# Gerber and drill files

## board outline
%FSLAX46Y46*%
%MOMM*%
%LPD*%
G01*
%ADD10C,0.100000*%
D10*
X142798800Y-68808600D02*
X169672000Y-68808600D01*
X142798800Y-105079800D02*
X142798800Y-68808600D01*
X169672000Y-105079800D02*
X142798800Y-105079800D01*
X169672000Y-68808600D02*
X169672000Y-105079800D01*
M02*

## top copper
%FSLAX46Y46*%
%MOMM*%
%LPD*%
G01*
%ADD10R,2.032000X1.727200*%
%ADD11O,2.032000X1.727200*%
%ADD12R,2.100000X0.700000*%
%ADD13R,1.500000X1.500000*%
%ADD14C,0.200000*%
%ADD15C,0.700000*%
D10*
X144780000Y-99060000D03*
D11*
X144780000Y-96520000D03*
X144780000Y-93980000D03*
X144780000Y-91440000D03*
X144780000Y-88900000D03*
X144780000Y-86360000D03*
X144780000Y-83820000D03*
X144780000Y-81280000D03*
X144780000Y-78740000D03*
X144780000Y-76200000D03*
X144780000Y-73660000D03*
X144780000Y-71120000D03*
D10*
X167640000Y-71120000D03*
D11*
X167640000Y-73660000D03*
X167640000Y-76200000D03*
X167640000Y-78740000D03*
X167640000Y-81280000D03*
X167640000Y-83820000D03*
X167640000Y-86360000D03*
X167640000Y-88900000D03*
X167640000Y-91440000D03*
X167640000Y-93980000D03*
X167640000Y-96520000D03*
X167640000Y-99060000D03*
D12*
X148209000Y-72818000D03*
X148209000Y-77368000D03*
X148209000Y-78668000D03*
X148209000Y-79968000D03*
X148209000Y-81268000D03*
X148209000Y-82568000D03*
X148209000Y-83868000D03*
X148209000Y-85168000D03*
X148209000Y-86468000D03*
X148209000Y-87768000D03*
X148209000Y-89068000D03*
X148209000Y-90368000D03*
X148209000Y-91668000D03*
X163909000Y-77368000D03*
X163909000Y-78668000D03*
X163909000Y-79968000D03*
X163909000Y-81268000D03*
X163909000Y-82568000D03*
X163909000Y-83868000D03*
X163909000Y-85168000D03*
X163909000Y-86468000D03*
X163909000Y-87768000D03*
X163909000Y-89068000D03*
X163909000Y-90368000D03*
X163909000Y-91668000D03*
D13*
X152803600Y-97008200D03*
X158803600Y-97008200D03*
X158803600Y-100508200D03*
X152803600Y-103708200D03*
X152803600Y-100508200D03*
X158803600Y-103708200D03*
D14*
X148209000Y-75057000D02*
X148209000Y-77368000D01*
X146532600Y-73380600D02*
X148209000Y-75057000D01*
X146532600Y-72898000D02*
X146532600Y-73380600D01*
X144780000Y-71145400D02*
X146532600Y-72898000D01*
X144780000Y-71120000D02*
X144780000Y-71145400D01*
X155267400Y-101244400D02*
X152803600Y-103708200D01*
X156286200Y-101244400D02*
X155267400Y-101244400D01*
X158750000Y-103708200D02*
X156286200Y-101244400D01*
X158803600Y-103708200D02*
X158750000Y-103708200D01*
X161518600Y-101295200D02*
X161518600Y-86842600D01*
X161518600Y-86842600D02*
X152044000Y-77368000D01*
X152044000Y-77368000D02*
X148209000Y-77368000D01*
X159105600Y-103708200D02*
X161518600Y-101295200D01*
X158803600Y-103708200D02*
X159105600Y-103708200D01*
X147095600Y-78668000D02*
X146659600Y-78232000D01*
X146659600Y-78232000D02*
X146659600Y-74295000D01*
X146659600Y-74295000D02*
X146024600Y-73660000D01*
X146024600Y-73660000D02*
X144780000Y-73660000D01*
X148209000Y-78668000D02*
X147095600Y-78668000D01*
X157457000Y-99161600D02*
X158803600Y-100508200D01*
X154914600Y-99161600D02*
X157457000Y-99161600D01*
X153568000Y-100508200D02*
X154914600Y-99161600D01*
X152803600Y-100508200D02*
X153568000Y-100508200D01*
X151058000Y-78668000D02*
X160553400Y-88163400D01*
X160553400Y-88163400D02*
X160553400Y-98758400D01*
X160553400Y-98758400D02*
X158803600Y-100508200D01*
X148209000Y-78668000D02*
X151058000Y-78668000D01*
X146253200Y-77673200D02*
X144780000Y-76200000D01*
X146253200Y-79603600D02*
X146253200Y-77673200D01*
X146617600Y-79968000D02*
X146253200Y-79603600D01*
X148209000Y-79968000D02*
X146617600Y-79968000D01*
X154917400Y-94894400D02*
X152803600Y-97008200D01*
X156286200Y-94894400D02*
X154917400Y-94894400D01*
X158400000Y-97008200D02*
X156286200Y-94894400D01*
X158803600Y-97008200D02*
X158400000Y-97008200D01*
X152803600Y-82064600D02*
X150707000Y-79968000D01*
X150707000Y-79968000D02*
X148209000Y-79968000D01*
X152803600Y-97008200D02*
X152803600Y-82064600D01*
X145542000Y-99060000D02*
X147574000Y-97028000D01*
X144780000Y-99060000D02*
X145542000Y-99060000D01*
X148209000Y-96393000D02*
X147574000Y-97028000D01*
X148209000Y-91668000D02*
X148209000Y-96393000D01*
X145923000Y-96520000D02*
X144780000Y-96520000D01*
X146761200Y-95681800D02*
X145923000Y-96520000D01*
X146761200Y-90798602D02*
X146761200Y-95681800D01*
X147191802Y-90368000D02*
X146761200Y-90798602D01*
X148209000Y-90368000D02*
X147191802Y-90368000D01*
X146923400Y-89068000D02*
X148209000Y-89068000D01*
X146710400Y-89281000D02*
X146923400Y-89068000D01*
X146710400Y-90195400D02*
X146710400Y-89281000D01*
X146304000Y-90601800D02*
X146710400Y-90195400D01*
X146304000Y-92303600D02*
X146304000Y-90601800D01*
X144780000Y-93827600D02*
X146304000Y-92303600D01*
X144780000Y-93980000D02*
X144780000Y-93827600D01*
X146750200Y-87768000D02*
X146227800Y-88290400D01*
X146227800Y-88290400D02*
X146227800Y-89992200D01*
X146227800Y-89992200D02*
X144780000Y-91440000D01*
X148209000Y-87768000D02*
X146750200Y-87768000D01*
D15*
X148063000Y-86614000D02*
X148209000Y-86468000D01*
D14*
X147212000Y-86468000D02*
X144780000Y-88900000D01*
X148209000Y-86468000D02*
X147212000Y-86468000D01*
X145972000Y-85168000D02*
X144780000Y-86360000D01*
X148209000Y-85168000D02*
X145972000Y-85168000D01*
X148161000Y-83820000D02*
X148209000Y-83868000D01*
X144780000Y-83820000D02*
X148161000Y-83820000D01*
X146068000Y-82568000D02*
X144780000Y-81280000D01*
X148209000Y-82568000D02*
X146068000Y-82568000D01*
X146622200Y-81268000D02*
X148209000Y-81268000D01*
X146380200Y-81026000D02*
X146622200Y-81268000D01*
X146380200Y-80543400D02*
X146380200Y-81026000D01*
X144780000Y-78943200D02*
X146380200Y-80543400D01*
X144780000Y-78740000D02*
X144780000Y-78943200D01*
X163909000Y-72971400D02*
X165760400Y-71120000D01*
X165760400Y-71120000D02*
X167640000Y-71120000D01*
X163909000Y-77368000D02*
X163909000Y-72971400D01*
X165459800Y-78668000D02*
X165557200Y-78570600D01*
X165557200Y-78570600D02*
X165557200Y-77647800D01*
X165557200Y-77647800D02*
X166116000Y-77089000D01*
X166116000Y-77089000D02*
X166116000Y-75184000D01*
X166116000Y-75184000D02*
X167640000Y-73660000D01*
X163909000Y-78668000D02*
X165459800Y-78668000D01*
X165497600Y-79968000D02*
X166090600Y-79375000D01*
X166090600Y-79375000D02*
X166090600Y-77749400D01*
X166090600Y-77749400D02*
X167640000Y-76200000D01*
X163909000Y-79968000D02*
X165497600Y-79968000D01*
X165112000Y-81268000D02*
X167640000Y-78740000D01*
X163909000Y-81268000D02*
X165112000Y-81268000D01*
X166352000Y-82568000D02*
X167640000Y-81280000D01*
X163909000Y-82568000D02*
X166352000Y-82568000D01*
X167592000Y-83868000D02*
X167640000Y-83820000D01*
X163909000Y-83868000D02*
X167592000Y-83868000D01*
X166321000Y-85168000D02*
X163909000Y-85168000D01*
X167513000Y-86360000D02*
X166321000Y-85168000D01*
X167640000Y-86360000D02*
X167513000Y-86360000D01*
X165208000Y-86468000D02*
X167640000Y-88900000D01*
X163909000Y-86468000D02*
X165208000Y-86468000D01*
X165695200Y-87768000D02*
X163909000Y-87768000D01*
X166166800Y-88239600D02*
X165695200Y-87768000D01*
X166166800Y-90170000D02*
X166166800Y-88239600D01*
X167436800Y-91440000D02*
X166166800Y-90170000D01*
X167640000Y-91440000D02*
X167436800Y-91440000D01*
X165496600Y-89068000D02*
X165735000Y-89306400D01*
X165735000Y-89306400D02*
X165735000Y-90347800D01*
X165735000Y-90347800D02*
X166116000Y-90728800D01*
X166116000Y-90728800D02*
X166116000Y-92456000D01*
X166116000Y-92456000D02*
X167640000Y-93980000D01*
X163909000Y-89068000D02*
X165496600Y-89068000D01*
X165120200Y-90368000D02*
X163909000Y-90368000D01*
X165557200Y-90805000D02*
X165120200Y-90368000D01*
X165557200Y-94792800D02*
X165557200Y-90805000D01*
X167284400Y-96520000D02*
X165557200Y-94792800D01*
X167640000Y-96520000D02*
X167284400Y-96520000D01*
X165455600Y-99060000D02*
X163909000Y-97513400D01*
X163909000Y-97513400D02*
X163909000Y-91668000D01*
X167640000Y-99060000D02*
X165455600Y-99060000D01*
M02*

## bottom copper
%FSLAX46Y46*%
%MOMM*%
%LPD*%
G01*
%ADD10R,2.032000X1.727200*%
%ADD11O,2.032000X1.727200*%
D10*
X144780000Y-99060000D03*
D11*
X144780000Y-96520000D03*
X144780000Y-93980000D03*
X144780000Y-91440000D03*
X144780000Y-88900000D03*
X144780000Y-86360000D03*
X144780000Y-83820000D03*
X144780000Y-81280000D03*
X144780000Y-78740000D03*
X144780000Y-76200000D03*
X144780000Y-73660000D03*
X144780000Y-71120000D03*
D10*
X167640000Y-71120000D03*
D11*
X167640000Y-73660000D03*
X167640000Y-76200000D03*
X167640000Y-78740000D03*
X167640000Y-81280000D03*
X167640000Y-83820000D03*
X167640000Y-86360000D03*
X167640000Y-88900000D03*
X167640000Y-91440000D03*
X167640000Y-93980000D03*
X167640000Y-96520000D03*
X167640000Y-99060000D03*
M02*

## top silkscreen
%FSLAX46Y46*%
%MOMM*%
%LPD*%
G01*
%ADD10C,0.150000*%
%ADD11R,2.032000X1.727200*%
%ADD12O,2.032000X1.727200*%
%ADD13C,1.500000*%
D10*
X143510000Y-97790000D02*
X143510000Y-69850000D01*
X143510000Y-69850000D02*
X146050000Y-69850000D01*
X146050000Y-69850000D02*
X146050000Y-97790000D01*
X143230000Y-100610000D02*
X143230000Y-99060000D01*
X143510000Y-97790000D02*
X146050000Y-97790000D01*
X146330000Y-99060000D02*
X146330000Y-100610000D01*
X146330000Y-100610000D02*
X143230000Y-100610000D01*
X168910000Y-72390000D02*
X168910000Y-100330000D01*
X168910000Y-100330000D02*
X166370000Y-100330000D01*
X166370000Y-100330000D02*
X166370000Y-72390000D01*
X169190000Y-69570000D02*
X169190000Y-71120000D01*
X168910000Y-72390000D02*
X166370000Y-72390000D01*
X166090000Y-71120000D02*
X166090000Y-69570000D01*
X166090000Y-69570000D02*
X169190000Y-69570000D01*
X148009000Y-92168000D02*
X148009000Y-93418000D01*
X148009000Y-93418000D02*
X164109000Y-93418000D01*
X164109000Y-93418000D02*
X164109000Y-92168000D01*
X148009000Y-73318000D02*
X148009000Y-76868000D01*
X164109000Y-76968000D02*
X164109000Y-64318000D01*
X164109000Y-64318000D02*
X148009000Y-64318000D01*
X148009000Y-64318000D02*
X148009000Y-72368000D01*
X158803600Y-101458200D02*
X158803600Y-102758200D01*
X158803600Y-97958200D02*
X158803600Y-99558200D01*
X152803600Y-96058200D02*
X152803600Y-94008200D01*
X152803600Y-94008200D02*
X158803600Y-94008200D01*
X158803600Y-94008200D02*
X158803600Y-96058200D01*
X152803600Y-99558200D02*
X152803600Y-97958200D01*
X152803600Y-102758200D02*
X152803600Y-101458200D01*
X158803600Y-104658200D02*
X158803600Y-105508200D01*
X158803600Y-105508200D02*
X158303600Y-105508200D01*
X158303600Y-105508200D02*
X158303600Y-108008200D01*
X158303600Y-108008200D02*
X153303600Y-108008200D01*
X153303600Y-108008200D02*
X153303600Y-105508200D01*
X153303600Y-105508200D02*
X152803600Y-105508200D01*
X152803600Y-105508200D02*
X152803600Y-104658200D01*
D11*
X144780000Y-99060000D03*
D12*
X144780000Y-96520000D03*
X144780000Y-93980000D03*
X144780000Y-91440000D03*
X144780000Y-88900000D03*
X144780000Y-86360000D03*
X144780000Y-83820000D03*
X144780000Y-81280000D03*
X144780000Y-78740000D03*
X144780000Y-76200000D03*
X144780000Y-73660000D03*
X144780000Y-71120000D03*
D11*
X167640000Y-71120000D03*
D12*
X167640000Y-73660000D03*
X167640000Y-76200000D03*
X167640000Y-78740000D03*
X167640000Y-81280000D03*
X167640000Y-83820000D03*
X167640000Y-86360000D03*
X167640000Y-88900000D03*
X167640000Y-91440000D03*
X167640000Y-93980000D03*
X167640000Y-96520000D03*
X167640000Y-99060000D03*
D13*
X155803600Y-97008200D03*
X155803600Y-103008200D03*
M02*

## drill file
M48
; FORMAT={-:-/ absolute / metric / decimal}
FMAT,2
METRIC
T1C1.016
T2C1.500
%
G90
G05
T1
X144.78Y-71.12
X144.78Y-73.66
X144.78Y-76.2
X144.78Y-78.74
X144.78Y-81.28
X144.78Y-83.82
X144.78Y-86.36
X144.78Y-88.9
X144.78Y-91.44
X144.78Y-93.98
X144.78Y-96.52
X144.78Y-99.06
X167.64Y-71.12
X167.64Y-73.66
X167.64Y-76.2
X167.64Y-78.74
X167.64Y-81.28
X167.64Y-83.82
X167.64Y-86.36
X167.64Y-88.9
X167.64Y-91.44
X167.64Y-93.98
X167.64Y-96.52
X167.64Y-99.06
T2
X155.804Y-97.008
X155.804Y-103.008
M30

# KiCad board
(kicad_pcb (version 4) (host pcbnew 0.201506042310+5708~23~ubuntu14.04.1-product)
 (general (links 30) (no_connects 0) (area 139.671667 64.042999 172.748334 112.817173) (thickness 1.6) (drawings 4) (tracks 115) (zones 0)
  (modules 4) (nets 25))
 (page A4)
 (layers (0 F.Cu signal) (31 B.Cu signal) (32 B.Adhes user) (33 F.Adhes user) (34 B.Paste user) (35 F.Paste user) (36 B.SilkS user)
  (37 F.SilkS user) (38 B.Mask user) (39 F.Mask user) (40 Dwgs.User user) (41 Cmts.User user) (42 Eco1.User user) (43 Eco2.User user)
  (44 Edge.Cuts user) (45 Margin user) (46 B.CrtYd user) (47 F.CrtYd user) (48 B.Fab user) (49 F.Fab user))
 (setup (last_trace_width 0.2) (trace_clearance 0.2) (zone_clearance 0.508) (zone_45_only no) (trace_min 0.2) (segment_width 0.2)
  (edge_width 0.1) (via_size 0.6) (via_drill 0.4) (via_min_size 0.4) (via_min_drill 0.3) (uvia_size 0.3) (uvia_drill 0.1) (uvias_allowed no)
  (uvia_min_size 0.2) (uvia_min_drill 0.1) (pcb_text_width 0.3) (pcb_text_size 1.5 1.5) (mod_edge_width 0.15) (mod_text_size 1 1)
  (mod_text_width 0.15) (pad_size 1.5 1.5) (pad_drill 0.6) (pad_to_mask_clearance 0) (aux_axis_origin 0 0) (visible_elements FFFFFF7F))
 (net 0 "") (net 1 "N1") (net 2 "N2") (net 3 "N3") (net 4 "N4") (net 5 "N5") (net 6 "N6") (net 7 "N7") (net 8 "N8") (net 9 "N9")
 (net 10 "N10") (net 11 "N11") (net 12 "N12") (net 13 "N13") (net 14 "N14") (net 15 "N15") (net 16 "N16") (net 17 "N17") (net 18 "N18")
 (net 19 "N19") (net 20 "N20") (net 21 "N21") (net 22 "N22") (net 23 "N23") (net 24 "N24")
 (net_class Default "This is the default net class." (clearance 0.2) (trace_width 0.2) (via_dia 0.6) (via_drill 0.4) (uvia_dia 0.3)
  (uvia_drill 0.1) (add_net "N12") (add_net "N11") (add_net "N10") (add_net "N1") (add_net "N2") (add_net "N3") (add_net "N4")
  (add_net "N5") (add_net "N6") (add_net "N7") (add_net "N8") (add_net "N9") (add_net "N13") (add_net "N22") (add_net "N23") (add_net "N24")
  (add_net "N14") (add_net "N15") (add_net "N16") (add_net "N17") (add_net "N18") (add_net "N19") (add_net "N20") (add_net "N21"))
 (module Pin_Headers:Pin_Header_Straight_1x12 (layer F.Cu) (at 144.78 99.06 180)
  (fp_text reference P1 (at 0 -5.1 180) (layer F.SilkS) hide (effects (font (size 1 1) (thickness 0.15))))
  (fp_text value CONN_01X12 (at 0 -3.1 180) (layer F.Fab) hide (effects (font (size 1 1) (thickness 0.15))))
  (fp_line (start 1.27 1.27) (end 1.27 29.21) (layer F.SilkS) (width 0.15))
  (fp_line (start 1.27 29.21) (end -1.27 29.21) (layer F.SilkS) (width 0.15))
  (fp_line (start -1.27 29.21) (end -1.27 1.27) (layer F.SilkS) (width 0.15))
  (fp_line (start 1.55 -1.55) (end 1.55 0) (layer F.SilkS) (width 0.15))
  (fp_line (start 1.27 1.27) (end -1.27 1.27) (layer F.SilkS) (width 0.15))
  (fp_line (start -1.55 0) (end -1.55 -1.55) (layer F.SilkS) (width 0.15))
  (fp_line (start -1.55 -1.55) (end 1.55 -1.55) (layer F.SilkS) (width 0.15))
  (pad 1 thru_hole rect (at 0 0 180) (size 2.032 1.7272) (drill 1.016) (layers *.Cu *.Mask F.SilkS) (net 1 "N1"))
  (pad 2 thru_hole oval (at 0 2.54 180) (size 2.032 1.7272) (drill 1.016) (layers *.Cu *.Mask F.SilkS) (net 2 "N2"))
  (pad 3 thru_hole oval (at 0 5.08 180) (size 2.032 1.7272) (drill 1.016) (layers *.Cu *.Mask F.SilkS) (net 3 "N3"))
  (pad 4 thru_hole oval (at 0 7.62 180) (size 2.032 1.7272) (drill 1.016) (layers *.Cu *.Mask F.SilkS) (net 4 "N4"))
  (pad 5 thru_hole oval (at 0 10.16 180) (size 2.032 1.7272) (drill 1.016) (layers *.Cu *.Mask F.SilkS) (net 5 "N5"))
  (pad 6 thru_hole oval (at 0 12.7 180) (size 2.032 1.7272) (drill 1.016) (layers *.Cu *.Mask F.SilkS) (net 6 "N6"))
  (pad 7 thru_hole oval (at 0 15.24 180) (size 2.032 1.7272) (drill 1.016) (layers *.Cu *.Mask F.SilkS) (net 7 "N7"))
  (pad 8 thru_hole oval (at 0 17.78 180) (size 2.032 1.7272) (drill 1.016) (layers *.Cu *.Mask F.SilkS) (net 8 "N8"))
  (pad 9 thru_hole oval (at 0 20.32 180) (size 2.032 1.7272) (drill 1.016) (layers *.Cu *.Mask F.SilkS) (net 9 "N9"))
  (pad 10 thru_hole oval (at 0 22.86 180) (size 2.032 1.7272) (drill 1.016) (layers *.Cu *.Mask F.SilkS) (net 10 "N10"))
  (pad 11 thru_hole oval (at 0 25.4 180) (size 2.032 1.7272) (drill 1.016) (layers *.Cu *.Mask F.SilkS) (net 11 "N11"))
  (pad 12 thru_hole oval (at 0 27.94 180) (size 2.032 1.7272) (drill 1.016) (layers *.Cu *.Mask F.SilkS) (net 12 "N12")))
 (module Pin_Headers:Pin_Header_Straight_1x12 (layer F.Cu) (at 167.64 71.12)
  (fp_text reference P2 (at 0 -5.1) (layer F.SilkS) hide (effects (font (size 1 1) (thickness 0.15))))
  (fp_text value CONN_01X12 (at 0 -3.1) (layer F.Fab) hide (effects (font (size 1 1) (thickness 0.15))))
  (fp_line (start 1.27 1.27) (end 1.27 29.21) (layer F.SilkS) (width 0.15))
  (fp_line (start 1.27 29.21) (end -1.27 29.21) (layer F.SilkS) (width 0.15))
  (fp_line (start -1.27 29.21) (end -1.27 1.27) (layer F.SilkS) (width 0.15))
  (fp_line (start 1.55 -1.55) (end 1.55 0) (layer F.SilkS) (width 0.15))
  (fp_line (start 1.27 1.27) (end -1.27 1.27) (layer F.SilkS) (width 0.15))
  (fp_line (start -1.55 0) (end -1.55 -1.55) (layer F.SilkS) (width 0.15))
  (fp_line (start -1.55 -1.55) (end 1.55 -1.55) (layer F.SilkS) (width 0.15))
  (pad 1 thru_hole rect (at 0 0) (size 2.032 1.7272) (drill 1.016) (layers *.Cu *.Mask F.SilkS) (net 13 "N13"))
  (pad 2 thru_hole oval (at 0 2.54) (size 2.032 1.7272) (drill 1.016) (layers *.Cu *.Mask F.SilkS) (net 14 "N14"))
  (pad 3 thru_hole oval (at 0 5.08) (size 2.032 1.7272) (drill 1.016) (layers *.Cu *.Mask F.SilkS) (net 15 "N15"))
  (pad 4 thru_hole oval (at 0 7.62) (size 2.032 1.7272) (drill 1.016) (layers *.Cu *.Mask F.SilkS) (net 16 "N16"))
  (pad 5 thru_hole oval (at 0 10.16) (size 2.032 1.7272) (drill 1.016) (layers *.Cu *.Mask F.SilkS) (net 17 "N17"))
  (pad 6 thru_hole oval (at 0 12.7) (size 2.032 1.7272) (drill 1.016) (layers *.Cu *.Mask F.SilkS) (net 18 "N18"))
  (pad 7 thru_hole oval (at 0 15.24) (size 2.032 1.7272) (drill 1.016) (layers *.Cu *.Mask F.SilkS) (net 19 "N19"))
  (pad 8 thru_hole oval (at 0 17.78) (size 2.032 1.7272) (drill 1.016) (layers *.Cu *.Mask F.SilkS) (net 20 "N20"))
  (pad 9 thru_hole oval (at 0 20.32) (size 2.032 1.7272) (drill 1.016) (layers *.Cu *.Mask F.SilkS) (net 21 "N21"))
  (pad 10 thru_hole oval (at 0 22.86) (size 2.032 1.7272) (drill 1.016) (layers *.Cu *.Mask F.SilkS) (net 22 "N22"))
  (pad 11 thru_hole oval (at 0 25.4) (size 2.032 1.7272) (drill 1.016) (layers *.Cu *.Mask F.SilkS) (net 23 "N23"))
  (pad 12 thru_hole oval (at 0 27.94) (size 2.032 1.7272) (drill 1.016) (layers *.Cu *.Mask F.SilkS) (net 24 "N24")))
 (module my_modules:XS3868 (layer F.Cu) (at 148.209 93.218)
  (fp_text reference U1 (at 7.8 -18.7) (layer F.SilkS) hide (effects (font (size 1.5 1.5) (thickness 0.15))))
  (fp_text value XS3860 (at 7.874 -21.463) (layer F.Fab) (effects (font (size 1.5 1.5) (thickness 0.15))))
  (fp_line (start -0.2 -1.05) (end -0.2 0.2) (layer F.SilkS) (width 0.15))
  (fp_line (start -0.2 0.2) (end 15.9 0.2) (layer F.SilkS) (width 0.15))
  (fp_line (start 15.9 0.2) (end 15.9 -1.05) (layer F.SilkS) (width 0.15))
  (fp_line (start -0.2 -19.9) (end -0.2 -16.35) (layer F.SilkS) (width 0.15))
  (fp_line (start 15.9 -16.25) (end 15.9 -28.9) (layer F.SilkS) (width 0.15))
  (fp_line (start 15.9 -28.9) (end -0.2 -28.9) (layer F.SilkS) (width 0.15))
  (fp_line (start -0.2 -28.9) (end -0.2 -20.85) (layer F.SilkS) (width 0.15))
  (pad 1 smd rect (at 0 -20.4) (size 2.1 0.7) (layers F.Cu F.Paste F.Mask))
  (pad 2 smd rect (at 0 -15.85) (size 2.1 0.7) (layers F.Cu F.Paste F.Mask) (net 12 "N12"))
  (pad 3 smd rect (at 0 -14.55) (size 2.1 0.7) (layers F.Cu F.Paste F.Mask) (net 11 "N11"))
  (pad 4 smd rect (at 0 -13.25) (size 2.1 0.7) (layers F.Cu F.Paste F.Mask) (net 10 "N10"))
  (pad 5 smd rect (at 0 -11.95) (size 2.1 0.7) (layers F.Cu F.Paste F.Mask) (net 9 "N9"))
  (pad 6 smd rect (at 0 -10.65) (size 2.1 0.7) (layers F.Cu F.Paste F.Mask) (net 8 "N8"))
  (pad 7 smd rect (at 0 -9.35) (size 2.1 0.7) (layers F.Cu F.Paste F.Mask) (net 7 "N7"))
  (pad 8 smd rect (at 0 -8.05) (size 2.1 0.7) (layers F.Cu F.Paste F.Mask) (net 6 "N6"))
  (pad 9 smd rect (at 0 -6.75) (size 2.1 0.7) (layers F.Cu F.Paste F.Mask) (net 5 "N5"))
  (pad 10 smd rect (at 0 -5.45) (size 2.1 0.7) (layers F.Cu F.Paste F.Mask) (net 4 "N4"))
  (pad 11 smd rect (at 0 -4.15) (size 2.1 0.7) (layers F.Cu F.Paste F.Mask) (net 3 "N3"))
  (pad 12 smd rect (at 0 -2.85) (size 2.1 0.7) (layers F.Cu F.Paste F.Mask) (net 2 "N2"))
  (pad 13 smd rect (at 0 -1.55) (size 2.1 0.7) (layers F.Cu F.Paste F.Mask) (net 1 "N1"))
  (pad 25 smd rect (at 15.7 -15.85) (size 2.1 0.7) (layers F.Cu F.Paste F.Mask) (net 13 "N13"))
  (pad 24 smd rect (at 15.7 -14.55) (size 2.1 0.7) (layers F.Cu F.Paste F.Mask) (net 14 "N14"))
  (pad 23 smd rect (at 15.7 -13.25) (size 2.1 0.7) (layers F.Cu F.Paste F.Mask) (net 15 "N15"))
  (pad 22 smd rect (at 15.7 -11.95) (size 2.1 0.7) (layers F.Cu F.Paste F.Mask) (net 16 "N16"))
  (pad 21 smd rect (at 15.7 -10.65) (size 2.1 0.7) (layers F.Cu F.Paste F.Mask) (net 17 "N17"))
  (pad 20 smd rect (at 15.7 -9.35) (size 2.1 0.7) (layers F.Cu F.Paste F.Mask) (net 18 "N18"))
  (pad 19 smd rect (at 15.7 -8.05) (size 2.1 0.7) (layers F.Cu F.Paste F.Mask) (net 19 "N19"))
  (pad 18 smd rect (at 15.7 -6.75) (size 2.1 0.7) (layers F.Cu F.Paste F.Mask) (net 20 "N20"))
  (pad 17 smd rect (at 15.7 -5.45) (size 2.1 0.7) (layers F.Cu F.Paste F.Mask) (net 21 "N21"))
  (pad 16 smd rect (at 15.7 -4.15) (size 2.1 0.7) (layers F.Cu F.Paste F.Mask) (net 22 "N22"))
  (pad 15 smd rect (at 15.7 -2.85) (size 2.1 0.7) (layers F.Cu F.Paste F.Mask) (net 23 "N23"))
  (pad 14 smd rect (at 15.7 -1.55) (size 2.1 0.7) (layers F.Cu F.Paste F.Mask) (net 24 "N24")))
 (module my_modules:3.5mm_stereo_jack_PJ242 (layer F.Cu) (at 155.8036 103.7082 180)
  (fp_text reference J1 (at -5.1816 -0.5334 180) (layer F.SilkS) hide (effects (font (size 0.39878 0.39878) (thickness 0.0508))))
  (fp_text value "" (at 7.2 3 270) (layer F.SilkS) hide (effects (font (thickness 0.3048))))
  (fp_line (start -3 2.25) (end -3 0.95) (layer F.SilkS) (width 0.15))
  (fp_line (start -3 5.75) (end -3 4.15) (layer F.SilkS) (width 0.15))
  (fp_line (start 3 7.65) (end 3 9.7) (layer F.SilkS) (width 0.15))
  (fp_line (start 3 9.7) (end -3 9.7) (layer F.SilkS) (width 0.15))
  (fp_line (start -3 9.7) (end -3 7.65) (layer F.SilkS) (width 0.15))
  (fp_line (start 3 4.15) (end 3 5.75) (layer F.SilkS) (width 0.15))
  (fp_line (start 3 0.95) (end 3 2.25) (layer F.SilkS) (width 0.15))
  (fp_line (start -3 -0.95) (end -3 -1.8) (layer F.SilkS) (width 0.15))
  (fp_line (start -3 -1.8) (end -2.5 -1.8) (layer F.SilkS) (width 0.15))
  (fp_line (start -2.5 -1.8) (end -2.5 -4.3) (layer F.SilkS) (width 0.15))
  (fp_line (start -2.5 -4.3) (end 2.5 -4.3) (layer F.SilkS) (width 0.15))
  (fp_line (start 2.5 -4.3) (end 2.5 -1.8) (layer F.SilkS) (width 0.15))
  (fp_line (start 2.5 -1.8) (end 3 -1.8) (layer F.SilkS) (width 0.15))
  (fp_line (start 3 -1.8) (end 3 -0.95) (layer F.SilkS) (width 0.15))
  (pad 5 smd rect (at 3 6.7 180) (size 1.5 1.5) (layers F.Cu F.Paste F.Mask) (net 10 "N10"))
  (pad 5 smd rect (at -3 6.7 180) (size 1.5 1.5) (layers F.Cu F.Paste F.Mask) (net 10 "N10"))
  (pad 2 smd rect (at -3 3.2 180) (size 1.5 1.5) (layers F.Cu F.Paste F.Mask) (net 11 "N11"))
  (pad 1 smd rect (at 3 0 180) (size 1.5 1.5) (layers F.Cu F.Paste F.Mask) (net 12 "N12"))
  (pad "" np_thru_hole circle (at 0 6.7 180) (size 1.5 1.5) (drill 1.5) (layers *.Cu *.Mask F.SilkS))
  (pad 2 smd rect (at 3 3.2 180) (size 1.5 1.5) (layers F.Cu F.Paste F.Mask) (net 11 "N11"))
  (pad 1 smd rect (at -3 0 180) (size 1.5 1.5) (layers F.Cu F.Paste F.Mask) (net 12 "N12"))
  (pad "" np_thru_hole circle (at 0 0.7 180) (size 1.5 1.5) (drill 1.5) (layers *.Cu *.Mask F.SilkS)))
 (gr_line (start 142.7988 68.8086) (end 169.672 68.8086) (angle 90) (layer Edge.Cuts) (width 0.1))
 (gr_line (start 142.7988 105.0798) (end 142.7988 68.8086) (angle 90) (layer Edge.Cuts) (width 0.1))
 (gr_line (start 169.672 105.0798) (end 142.7988 105.0798) (angle 90) (layer Edge.Cuts) (width 0.1))
 (gr_line (start 169.672 68.8086) (end 169.672 105.0798) (angle 90) (layer Edge.Cuts) (width 0.1))
 (segment (start 148.209 75.057) (end 148.209 77.368) (width 0.2) (layer F.Cu) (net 12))
 (segment (start 146.5326 73.3806) (end 148.209 75.057) (width 0.2) (layer F.Cu) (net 12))
 (segment (start 146.5326 72.898) (end 146.5326 73.3806) (width 0.2) (layer F.Cu) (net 12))
 (segment (start 144.78 71.1454) (end 146.5326 72.898) (width 0.2) (layer F.Cu) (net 12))
 (segment (start 144.78 71.12) (end 144.78 71.1454) (width 0.2) (layer F.Cu) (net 12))
 (segment (start 155.2674 101.2444) (end 152.8036 103.7082) (width 0.2) (layer F.Cu) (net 12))
 (segment (start 156.2862 101.2444) (end 155.2674 101.2444) (width 0.2) (layer F.Cu) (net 12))
 (segment (start 158.75 103.7082) (end 156.2862 101.2444) (width 0.2) (layer F.Cu) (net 12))
 (segment (start 158.8036 103.7082) (end 158.75 103.7082) (width 0.2) (layer F.Cu) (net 12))
 (segment (start 161.5186 101.2952) (end 161.5186 86.8426) (width 0.2) (layer F.Cu) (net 12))
 (segment (start 161.5186 86.8426) (end 152.044 77.368) (width 0.2) (layer F.Cu) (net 12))
 (segment (start 152.044 77.368) (end 148.209 77.368) (width 0.2) (layer F.Cu) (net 12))
 (segment (start 159.1056 103.7082) (end 161.5186 101.2952) (width 0.2) (layer F.Cu) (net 12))
 (segment (start 158.8036 103.7082) (end 159.1056 103.7082) (width 0.2) (layer F.Cu) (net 12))
 (segment (start 147.0956 78.668) (end 146.6596 78.232) (width 0.2) (layer F.Cu) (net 11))
 (segment (start 146.6596 78.232) (end 146.6596 74.295) (width 0.2) (layer F.Cu) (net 11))
 (segment (start 146.6596 74.295) (end 146.0246 73.66) (width 0.2) (layer F.Cu) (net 11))
 (segment (start 146.0246 73.66) (end 144.78 73.66) (width 0.2) (layer F.Cu) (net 11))
 (segment (start 148.209 78.668) (end 147.0956 78.668) (width 0.2) (layer F.Cu) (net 11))
 (segment (start 157.457 99.1616) (end 158.8036 100.5082) (width 0.2) (layer F.Cu) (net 11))
 (segment (start 154.9146 99.1616) (end 157.457 99.1616) (width 0.2) (layer F.Cu) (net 11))
 (segment (start 153.568 100.5082) (end 154.9146 99.1616) (width 0.2) (layer F.Cu) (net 11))
 (segment (start 152.8036 100.5082) (end 153.568 100.5082) (width 0.2) (layer F.Cu) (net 11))
 (segment (start 151.058 78.668) (end 160.5534 88.1634) (width 0.2) (layer F.Cu) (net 11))
 (segment (start 160.5534 88.1634) (end 160.5534 98.7584) (width 0.2) (layer F.Cu) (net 11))
 (segment (start 160.5534 98.7584) (end 158.8036 100.5082) (width 0.2) (layer F.Cu) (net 11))
 (segment (start 148.209 78.668) (end 151.058 78.668) (width 0.2) (layer F.Cu) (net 11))
 (segment (start 146.2532 77.6732) (end 144.78 76.2) (width 0.2) (layer F.Cu) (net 10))
 (segment (start 146.2532 79.6036) (end 146.2532 77.6732) (width 0.2) (layer F.Cu) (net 10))
 (segment (start 146.6176 79.968) (end 146.2532 79.6036) (width 0.2) (layer F.Cu) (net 10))
 (segment (start 148.209 79.968) (end 146.6176 79.968) (width 0.2) (layer F.Cu) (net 10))
 (segment (start 154.9174 94.8944) (end 152.8036 97.0082) (width 0.2) (layer F.Cu) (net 10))
 (segment (start 156.2862 94.8944) (end 154.9174 94.8944) (width 0.2) (layer F.Cu) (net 10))
 (segment (start 158.4 97.0082) (end 156.2862 94.8944) (width 0.2) (layer F.Cu) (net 10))
 (segment (start 158.8036 97.0082) (end 158.4 97.0082) (width 0.2) (layer F.Cu) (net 10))
 (segment (start 152.8036 82.0646) (end 150.707 79.968) (width 0.2) (layer F.Cu) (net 10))
 (segment (start 150.707 79.968) (end 148.209 79.968) (width 0.2) (layer F.Cu) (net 10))
 (segment (start 152.8036 97.0082) (end 152.8036 82.0646) (width 0.2) (layer F.Cu) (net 10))
 (segment (start 145.542 99.06) (end 147.574 97.028) (width 0.2) (layer F.Cu) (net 1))
 (segment (start 144.78 99.06) (end 145.542 99.06) (width 0.2) (layer F.Cu) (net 1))
 (segment (start 148.209 96.393) (end 147.574 97.028) (width 0.2) (layer F.Cu) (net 1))
 (segment (start 148.209 91.668) (end 148.209 96.393) (width 0.2) (layer F.Cu) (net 1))
 (segment (start 145.923 96.52) (end 144.78 96.52) (width 0.2) (layer F.Cu) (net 2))
 (segment (start 146.7612 95.6818) (end 145.923 96.52) (width 0.2) (layer F.Cu) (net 2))
 (segment (start 146.7612 90.798602) (end 146.7612 95.6818) (width 0.2) (layer F.Cu) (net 2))
 (segment (start 147.191802 90.368) (end 146.7612 90.798602) (width 0.2) (layer F.Cu) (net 2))
 (segment (start 148.209 90.368) (end 147.191802 90.368) (width 0.2) (layer F.Cu) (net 2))
 (segment (start 146.9234 89.068) (end 148.209 89.068) (width 0.2) (layer F.Cu) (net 3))
 (segment (start 146.7104 89.281) (end 146.9234 89.068) (width 0.2) (layer F.Cu) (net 3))
 (segment (start 146.7104 90.1954) (end 146.7104 89.281) (width 0.2) (layer F.Cu) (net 3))
 (segment (start 146.304 90.6018) (end 146.7104 90.1954) (width 0.2) (layer F.Cu) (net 3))
 (segment (start 146.304 92.3036) (end 146.304 90.6018) (width 0.2) (layer F.Cu) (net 3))
 (segment (start 144.78 93.8276) (end 146.304 92.3036) (width 0.2) (layer F.Cu) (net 3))
 (segment (start 144.78 93.98) (end 144.78 93.8276) (width 0.2) (layer F.Cu) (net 3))
 (segment (start 146.7502 87.768) (end 146.2278 88.2904) (width 0.2) (layer F.Cu) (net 4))
 (segment (start 146.2278 88.2904) (end 146.2278 89.9922) (width 0.2) (layer F.Cu) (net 4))
 (segment (start 146.2278 89.9922) (end 144.78 91.44) (width 0.2) (layer F.Cu) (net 4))
 (segment (start 148.209 87.768) (end 146.7502 87.768) (width 0.2) (layer F.Cu) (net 4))
 (segment (start 148.063 86.614) (end 148.209 86.468) (width 0.7) (layer F.Cu) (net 5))
 (segment (start 147.212 86.468) (end 144.78 88.9) (width 0.2) (layer F.Cu) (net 5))
 (segment (start 148.209 86.468) (end 147.212 86.468) (width 0.2) (layer F.Cu) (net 5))
 (segment (start 145.972 85.168) (end 144.78 86.36) (width 0.2) (layer F.Cu) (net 6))
 (segment (start 148.209 85.168) (end 145.972 85.168) (width 0.2) (layer F.Cu) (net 6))
 (segment (start 148.161 83.82) (end 148.209 83.868) (width 0.2) (layer F.Cu) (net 7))
 (segment (start 144.78 83.82) (end 148.161 83.82) (width 0.2) (layer F.Cu) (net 7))
 (segment (start 146.068 82.568) (end 144.78 81.28) (width 0.2) (layer F.Cu) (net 8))
 (segment (start 148.209 82.568) (end 146.068 82.568) (width 0.2) (layer F.Cu) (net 8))
 (segment (start 146.6222 81.268) (end 148.209 81.268) (width 0.2) (layer F.Cu) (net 9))
 (segment (start 146.3802 81.026) (end 146.6222 81.268) (width 0.2) (layer F.Cu) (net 9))
 (segment (start 146.3802 80.5434) (end 146.3802 81.026) (width 0.2) (layer F.Cu) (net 9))
 (segment (start 144.78 78.9432) (end 146.3802 80.5434) (width 0.2) (layer F.Cu) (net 9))
 (segment (start 144.78 78.74) (end 144.78 78.9432) (width 0.2) (layer F.Cu) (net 9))
 (segment (start 163.909 72.9714) (end 165.7604 71.12) (width 0.2) (layer F.Cu) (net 13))
 (segment (start 165.7604 71.12) (end 167.64 71.12) (width 0.2) (layer F.Cu) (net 13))
 (segment (start 163.909 77.368) (end 163.909 72.9714) (width 0.2) (layer F.Cu) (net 13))
 (segment (start 165.4598 78.668) (end 165.5572 78.5706) (width 0.2) (layer F.Cu) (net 14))
 (segment (start 165.5572 78.5706) (end 165.5572 77.6478) (width 0.2) (layer F.Cu) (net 14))
 (segment (start 165.5572 77.6478) (end 166.116 77.089) (width 0.2) (layer F.Cu) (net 14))
 (segment (start 166.116 77.089) (end 166.116 75.184) (width 0.2) (layer F.Cu) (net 14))
 (segment (start 166.116 75.184) (end 167.64 73.66) (width 0.2) (layer F.Cu) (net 14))
 (segment (start 163.909 78.668) (end 165.4598 78.668) (width 0.2) (layer F.Cu) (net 14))
 (segment (start 165.4976 79.968) (end 166.0906 79.375) (width 0.2) (layer F.Cu) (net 15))
 (segment (start 166.0906 79.375) (end 166.0906 77.7494) (width 0.2) (layer F.Cu) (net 15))
 (segment (start 166.0906 77.7494) (end 167.64 76.2) (width 0.2) (layer F.Cu) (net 15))
 (segment (start 163.909 79.968) (end 165.4976 79.968) (width 0.2) (layer F.Cu) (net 15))
 (segment (start 165.112 81.268) (end 167.64 78.74) (width 0.2) (layer F.Cu) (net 16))
 (segment (start 163.909 81.268) (end 165.112 81.268) (width 0.2) (layer F.Cu) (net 16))
 (segment (start 166.352 82.568) (end 167.64 81.28) (width 0.2) (layer F.Cu) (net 17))
 (segment (start 163.909 82.568) (end 166.352 82.568) (width 0.2) (layer F.Cu) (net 17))
 (segment (start 167.592 83.868) (end 167.64 83.82) (width 0.2) (layer F.Cu) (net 18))
 (segment (start 163.909 83.868) (end 167.592 83.868) (width 0.2) (layer F.Cu) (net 18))
 (segment (start 166.321 85.168) (end 163.909 85.168) (width 0.2) (layer F.Cu) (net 19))
 (segment (start 167.513 86.36) (end 166.321 85.168) (width 0.2) (layer F.Cu) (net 19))
 (segment (start 167.64 86.36) (end 167.513 86.36) (width 0.2) (layer F.Cu) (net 19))
 (segment (start 165.208 86.468) (end 167.64 88.9) (width 0.2) (layer F.Cu) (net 20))
 (segment (start 163.909 86.468) (end 165.208 86.468) (width 0.2) (layer F.Cu) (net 20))
 (segment (start 165.6952 87.768) (end 163.909 87.768) (width 0.2) (layer F.Cu) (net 21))
 (segment (start 166.1668 88.2396) (end 165.6952 87.768) (width 0.2) (layer F.Cu) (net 21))
 (segment (start 166.1668 90.17) (end 166.1668 88.2396) (width 0.2) (layer F.Cu) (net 21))
 (segment (start 167.4368 91.44) (end 166.1668 90.17) (width 0.2) (layer F.Cu) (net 21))
 (segment (start 167.64 91.44) (end 167.4368 91.44) (width 0.2) (layer F.Cu) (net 21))
 (segment (start 165.4966 89.068) (end 165.735 89.3064) (width 0.2) (layer F.Cu) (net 22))
 (segment (start 165.735 89.3064) (end 165.735 90.3478) (width 0.2) (layer F.Cu) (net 22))
 (segment (start 165.735 90.3478) (end 166.116 90.7288) (width 0.2) (layer F.Cu) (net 22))
 (segment (start 166.116 90.7288) (end 166.116 92.456) (width 0.2) (layer F.Cu) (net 22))
 (segment (start 166.116 92.456) (end 167.64 93.98) (width 0.2) (layer F.Cu) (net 22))
 (segment (start 163.909 89.068) (end 165.4966 89.068) (width 0.2) (layer F.Cu) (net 22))
 (segment (start 165.1202 90.368) (end 163.909 90.368) (width 0.2) (layer F.Cu) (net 23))
 (segment (start 165.5572 90.805) (end 165.1202 90.368) (width 0.2) (layer F.Cu) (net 23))
 (segment (start 165.5572 94.7928) (end 165.5572 90.805) (width 0.2) (layer F.Cu) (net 23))
 (segment (start 167.2844 96.52) (end 165.5572 94.7928) (width 0.2) (layer F.Cu) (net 23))
 (segment (start 167.64 96.52) (end 167.2844 96.52) (width 0.2) (layer F.Cu) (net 23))
 (segment (start 165.4556 99.06) (end 163.909 97.5134) (width 0.2) (layer F.Cu) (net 24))
 (segment (start 163.909 97.5134) (end 163.909 91.668) (width 0.2) (layer F.Cu) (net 24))
 (segment (start 167.64 99.06) (end 165.4556 99.06) (width 0.2) (layer F.Cu) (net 24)))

